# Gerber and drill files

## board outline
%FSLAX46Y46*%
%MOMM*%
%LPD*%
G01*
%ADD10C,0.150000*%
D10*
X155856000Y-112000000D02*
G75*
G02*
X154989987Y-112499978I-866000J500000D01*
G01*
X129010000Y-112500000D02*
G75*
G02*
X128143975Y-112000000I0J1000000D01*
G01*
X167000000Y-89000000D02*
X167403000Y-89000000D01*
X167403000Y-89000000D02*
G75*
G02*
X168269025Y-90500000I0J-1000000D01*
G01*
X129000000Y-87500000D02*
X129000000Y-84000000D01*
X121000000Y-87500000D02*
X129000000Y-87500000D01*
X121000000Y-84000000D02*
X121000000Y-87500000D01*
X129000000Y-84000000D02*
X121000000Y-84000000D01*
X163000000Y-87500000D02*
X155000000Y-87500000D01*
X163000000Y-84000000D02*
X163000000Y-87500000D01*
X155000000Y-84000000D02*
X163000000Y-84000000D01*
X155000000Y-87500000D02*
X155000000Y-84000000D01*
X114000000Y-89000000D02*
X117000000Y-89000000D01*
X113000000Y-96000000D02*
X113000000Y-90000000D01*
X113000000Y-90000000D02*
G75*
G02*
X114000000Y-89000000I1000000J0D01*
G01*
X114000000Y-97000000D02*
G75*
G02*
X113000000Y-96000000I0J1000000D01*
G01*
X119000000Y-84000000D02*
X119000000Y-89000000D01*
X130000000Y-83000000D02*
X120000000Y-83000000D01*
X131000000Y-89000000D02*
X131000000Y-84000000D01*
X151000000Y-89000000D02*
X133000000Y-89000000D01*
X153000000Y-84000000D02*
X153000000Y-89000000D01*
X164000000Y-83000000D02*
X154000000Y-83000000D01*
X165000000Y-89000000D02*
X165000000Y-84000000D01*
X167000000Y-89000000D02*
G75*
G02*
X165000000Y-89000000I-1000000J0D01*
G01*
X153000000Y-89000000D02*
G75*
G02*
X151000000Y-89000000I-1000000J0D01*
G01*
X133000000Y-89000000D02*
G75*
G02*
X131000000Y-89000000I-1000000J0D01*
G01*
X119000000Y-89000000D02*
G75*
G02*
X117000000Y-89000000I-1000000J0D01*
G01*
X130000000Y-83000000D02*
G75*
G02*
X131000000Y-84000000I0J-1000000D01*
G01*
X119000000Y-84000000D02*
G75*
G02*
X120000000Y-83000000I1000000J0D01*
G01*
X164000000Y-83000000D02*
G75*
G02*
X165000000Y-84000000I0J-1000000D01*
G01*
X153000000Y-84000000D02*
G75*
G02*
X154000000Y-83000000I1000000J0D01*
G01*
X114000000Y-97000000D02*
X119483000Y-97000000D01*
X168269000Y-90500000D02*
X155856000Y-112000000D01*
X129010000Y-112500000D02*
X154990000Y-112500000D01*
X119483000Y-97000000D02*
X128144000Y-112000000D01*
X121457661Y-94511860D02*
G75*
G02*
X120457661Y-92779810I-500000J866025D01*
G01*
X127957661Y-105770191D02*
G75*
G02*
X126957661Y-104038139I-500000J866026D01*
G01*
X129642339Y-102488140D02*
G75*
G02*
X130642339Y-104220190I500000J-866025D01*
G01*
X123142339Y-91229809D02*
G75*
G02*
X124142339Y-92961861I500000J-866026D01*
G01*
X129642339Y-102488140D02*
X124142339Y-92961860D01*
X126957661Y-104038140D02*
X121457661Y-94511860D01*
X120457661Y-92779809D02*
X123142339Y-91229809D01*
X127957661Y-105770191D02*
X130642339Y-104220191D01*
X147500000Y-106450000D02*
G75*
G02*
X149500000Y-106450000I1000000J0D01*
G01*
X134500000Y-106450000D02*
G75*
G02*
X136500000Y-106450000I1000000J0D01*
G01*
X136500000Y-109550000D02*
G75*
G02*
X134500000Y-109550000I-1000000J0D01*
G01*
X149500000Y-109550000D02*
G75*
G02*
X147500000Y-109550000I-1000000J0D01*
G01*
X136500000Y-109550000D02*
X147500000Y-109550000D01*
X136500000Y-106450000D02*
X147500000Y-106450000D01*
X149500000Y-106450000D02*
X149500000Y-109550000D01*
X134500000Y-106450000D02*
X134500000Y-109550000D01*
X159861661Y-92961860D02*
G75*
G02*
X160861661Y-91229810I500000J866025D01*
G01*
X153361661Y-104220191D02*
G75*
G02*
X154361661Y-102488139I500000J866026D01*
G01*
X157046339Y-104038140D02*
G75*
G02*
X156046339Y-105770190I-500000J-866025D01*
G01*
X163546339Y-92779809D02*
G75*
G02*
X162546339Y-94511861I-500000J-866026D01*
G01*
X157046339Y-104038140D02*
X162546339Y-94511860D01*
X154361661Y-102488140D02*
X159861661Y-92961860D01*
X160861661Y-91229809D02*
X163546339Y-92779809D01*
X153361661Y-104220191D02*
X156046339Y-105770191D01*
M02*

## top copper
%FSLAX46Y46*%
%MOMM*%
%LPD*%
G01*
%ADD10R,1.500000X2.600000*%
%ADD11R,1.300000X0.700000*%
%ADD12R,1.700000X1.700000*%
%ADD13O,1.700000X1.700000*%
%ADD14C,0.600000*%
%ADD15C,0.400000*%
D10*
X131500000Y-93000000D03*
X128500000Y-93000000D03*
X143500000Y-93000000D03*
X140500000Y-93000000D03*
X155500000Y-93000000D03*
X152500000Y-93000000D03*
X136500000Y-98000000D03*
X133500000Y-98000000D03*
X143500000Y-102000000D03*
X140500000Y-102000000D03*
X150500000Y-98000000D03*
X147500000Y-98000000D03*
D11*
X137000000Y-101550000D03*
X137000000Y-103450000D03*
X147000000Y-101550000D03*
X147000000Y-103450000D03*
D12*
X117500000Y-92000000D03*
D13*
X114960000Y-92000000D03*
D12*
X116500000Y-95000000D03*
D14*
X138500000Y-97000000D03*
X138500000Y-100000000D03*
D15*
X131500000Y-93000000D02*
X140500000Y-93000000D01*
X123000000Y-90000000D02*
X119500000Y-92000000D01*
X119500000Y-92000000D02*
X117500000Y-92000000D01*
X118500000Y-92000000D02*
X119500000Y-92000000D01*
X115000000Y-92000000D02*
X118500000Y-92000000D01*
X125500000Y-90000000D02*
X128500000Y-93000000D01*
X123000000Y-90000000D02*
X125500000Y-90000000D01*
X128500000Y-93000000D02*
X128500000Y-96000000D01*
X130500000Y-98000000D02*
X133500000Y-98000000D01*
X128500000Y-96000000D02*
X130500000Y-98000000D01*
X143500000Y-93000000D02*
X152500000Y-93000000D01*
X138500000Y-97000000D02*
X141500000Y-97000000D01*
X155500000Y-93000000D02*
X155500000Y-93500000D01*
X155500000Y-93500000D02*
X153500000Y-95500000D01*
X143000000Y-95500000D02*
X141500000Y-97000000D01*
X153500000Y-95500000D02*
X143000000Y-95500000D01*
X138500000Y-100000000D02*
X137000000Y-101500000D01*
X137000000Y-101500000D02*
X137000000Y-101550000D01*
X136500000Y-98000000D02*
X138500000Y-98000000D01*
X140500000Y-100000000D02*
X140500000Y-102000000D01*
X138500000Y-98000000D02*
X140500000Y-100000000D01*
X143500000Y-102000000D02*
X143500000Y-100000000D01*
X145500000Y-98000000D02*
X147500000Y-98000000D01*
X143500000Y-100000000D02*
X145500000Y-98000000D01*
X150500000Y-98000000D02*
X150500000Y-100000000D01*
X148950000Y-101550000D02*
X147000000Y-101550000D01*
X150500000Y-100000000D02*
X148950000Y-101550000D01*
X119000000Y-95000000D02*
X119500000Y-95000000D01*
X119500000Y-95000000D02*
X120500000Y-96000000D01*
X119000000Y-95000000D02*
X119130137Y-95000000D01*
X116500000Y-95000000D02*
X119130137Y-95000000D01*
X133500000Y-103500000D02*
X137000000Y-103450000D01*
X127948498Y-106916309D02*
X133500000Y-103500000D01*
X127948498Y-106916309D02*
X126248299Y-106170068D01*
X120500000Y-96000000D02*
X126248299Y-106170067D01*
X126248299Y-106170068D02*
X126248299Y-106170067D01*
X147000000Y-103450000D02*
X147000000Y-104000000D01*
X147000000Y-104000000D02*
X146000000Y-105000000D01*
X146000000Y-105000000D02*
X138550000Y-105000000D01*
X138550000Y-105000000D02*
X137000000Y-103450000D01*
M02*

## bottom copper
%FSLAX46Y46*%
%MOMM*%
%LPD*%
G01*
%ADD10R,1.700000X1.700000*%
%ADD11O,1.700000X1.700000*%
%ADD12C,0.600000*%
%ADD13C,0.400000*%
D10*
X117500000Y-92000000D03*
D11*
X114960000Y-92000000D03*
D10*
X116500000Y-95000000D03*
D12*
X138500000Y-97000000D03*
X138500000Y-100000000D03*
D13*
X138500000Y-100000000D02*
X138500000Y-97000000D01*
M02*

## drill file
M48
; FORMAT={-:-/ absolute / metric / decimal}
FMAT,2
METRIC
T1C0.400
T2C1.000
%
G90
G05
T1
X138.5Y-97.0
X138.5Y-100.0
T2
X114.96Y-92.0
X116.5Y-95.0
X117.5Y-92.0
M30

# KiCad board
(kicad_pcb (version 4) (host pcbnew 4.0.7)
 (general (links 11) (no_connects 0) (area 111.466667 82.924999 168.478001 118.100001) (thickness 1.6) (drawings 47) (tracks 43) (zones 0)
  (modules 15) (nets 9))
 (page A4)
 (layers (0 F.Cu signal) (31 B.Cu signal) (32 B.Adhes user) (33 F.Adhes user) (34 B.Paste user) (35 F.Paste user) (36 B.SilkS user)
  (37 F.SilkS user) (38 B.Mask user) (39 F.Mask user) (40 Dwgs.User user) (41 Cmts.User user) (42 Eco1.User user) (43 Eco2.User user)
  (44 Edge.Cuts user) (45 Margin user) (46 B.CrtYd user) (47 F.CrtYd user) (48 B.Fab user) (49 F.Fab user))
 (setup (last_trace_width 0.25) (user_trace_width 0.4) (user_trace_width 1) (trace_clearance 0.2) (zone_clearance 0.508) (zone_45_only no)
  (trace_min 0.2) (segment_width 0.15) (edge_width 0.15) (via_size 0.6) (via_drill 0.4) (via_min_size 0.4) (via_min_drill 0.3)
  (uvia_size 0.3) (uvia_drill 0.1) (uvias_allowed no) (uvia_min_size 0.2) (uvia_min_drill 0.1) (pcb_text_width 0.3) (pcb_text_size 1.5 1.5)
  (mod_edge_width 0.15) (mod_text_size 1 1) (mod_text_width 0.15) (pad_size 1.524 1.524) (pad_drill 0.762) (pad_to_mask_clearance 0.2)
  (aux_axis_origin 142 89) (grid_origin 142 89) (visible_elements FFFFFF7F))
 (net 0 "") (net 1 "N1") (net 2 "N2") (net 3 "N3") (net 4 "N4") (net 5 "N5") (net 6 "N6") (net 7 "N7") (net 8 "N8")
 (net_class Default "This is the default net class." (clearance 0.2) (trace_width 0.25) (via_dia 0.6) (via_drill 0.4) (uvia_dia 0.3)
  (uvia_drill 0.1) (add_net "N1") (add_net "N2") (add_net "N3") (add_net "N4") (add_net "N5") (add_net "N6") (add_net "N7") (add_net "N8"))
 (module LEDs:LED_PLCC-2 (layer F.Cu) (at 130 93 180)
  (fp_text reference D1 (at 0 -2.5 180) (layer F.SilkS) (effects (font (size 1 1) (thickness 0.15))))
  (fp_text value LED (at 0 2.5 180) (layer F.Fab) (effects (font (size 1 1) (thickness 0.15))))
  (pad 1 smd rect (at -1.5 0 180) (size 1.5 2.6) (layers F.Cu F.Paste F.Mask) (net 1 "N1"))
  (pad 2 smd rect (at 1.5 0 180) (size 1.5 2.6) (layers F.Cu F.Paste F.Mask) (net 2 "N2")))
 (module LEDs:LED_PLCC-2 (layer F.Cu) (at 142 93 180)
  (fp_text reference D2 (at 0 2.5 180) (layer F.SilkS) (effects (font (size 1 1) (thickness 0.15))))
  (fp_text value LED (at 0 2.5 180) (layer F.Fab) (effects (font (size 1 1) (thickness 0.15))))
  (pad 1 smd rect (at -1.5 0 180) (size 1.5 2.6) (layers F.Cu F.Paste F.Mask) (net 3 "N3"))
  (pad 2 smd rect (at 1.5 0 180) (size 1.5 2.6) (layers F.Cu F.Paste F.Mask) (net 1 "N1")))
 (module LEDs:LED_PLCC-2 (layer F.Cu) (at 154 93 180)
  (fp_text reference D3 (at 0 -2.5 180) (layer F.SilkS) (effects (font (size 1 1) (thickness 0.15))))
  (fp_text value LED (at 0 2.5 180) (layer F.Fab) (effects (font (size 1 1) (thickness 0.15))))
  (pad 1 smd rect (at -1.5 0 180) (size 1.5 2.6) (layers F.Cu F.Paste F.Mask) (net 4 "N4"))
  (pad 2 smd rect (at 1.5 0 180) (size 1.5 2.6) (layers F.Cu F.Paste F.Mask) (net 3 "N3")))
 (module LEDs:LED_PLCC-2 (layer F.Cu) (at 135 98 180)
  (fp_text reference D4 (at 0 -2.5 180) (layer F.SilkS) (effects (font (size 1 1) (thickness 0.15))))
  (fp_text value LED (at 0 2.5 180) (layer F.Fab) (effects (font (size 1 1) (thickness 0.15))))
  (pad 1 smd rect (at -1.5 0 180) (size 1.5 2.6) (layers F.Cu F.Paste F.Mask) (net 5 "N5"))
  (pad 2 smd rect (at 1.5 0 180) (size 1.5 2.6) (layers F.Cu F.Paste F.Mask) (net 2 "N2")))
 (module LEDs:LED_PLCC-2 (layer F.Cu) (at 142 102 180)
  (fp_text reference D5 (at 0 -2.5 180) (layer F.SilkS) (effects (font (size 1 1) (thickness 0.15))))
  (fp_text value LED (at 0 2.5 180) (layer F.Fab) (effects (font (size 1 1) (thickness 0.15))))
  (pad 1 smd rect (at -1.5 0 180) (size 1.5 2.6) (layers F.Cu F.Paste F.Mask) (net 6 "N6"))
  (pad 2 smd rect (at 1.5 0 180) (size 1.5 2.6) (layers F.Cu F.Paste F.Mask) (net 5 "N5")))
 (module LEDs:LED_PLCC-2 (layer F.Cu) (at 149 98 180)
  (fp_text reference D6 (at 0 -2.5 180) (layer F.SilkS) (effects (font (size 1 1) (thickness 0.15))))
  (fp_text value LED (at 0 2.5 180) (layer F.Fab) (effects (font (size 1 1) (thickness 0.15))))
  (pad 1 smd rect (at -1.5 0 180) (size 1.5 2.6) (layers F.Cu F.Paste F.Mask) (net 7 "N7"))
  (pad 2 smd rect (at 1.5 0 180) (size 1.5 2.6) (layers F.Cu F.Paste F.Mask) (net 6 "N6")))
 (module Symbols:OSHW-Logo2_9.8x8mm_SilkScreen (layer B.Cu) (at 142 100 180)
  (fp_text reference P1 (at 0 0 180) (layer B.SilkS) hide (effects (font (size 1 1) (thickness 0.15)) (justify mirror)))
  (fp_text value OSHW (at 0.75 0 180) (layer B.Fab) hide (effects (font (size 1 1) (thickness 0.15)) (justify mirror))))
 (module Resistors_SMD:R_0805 (layer F.Cu) (at 137 102.5 270)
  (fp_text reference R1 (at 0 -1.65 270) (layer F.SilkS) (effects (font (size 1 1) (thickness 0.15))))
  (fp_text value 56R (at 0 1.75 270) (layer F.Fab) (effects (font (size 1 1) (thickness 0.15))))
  (pad 1 smd rect (at -0.95 0 270) (size 0.7 1.3) (layers F.Cu F.Paste F.Mask) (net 4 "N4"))
  (pad 2 smd rect (at 0.95 0 270) (size 0.7 1.3) (layers F.Cu F.Paste F.Mask) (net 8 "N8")))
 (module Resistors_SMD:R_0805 (layer F.Cu) (at 147 102.5 270)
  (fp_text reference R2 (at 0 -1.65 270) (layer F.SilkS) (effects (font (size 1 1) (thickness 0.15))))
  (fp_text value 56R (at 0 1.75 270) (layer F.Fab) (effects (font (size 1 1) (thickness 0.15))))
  (pad 1 smd rect (at -0.95 0 270) (size 0.7 1.3) (layers F.Cu F.Paste F.Mask) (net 7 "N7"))
  (pad 2 smd rect (at 0.95 0 270) (size 0.7 1.3) (layers F.Cu F.Paste F.Mask) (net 8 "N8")))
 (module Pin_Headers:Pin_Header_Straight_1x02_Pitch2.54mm (layer F.Cu) (at 117.5 92 270)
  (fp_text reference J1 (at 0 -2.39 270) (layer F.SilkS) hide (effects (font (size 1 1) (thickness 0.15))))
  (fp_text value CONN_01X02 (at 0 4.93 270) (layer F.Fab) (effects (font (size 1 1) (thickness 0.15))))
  (pad 1 thru_hole rect (at 0 0 270) (size 1.7 1.7) (drill 1) (layers *.Cu *.Mask) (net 2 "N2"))
  (pad 2 thru_hole oval (at 0 2.54 270) (size 1.7 1.7) (drill 1) (layers *.Cu *.Mask) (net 2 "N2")))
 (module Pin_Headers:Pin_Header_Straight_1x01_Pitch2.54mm (layer F.Cu) (at 116.5 95)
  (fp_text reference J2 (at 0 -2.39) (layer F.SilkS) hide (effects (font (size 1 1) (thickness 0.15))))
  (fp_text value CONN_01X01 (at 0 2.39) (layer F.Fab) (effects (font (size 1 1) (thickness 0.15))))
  (pad 1 thru_hole rect (at 0 0) (size 1.7 1.7) (drill 1) (layers *.Cu *.Mask) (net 8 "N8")))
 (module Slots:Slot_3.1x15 (layer F.Cu) (at 125.55 98.5 120)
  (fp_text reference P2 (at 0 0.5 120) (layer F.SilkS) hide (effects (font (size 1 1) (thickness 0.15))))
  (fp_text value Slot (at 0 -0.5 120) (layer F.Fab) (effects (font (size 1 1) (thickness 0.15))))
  (fp_arc (start 6.5 -1.55) (end 5.5 -1.55) (angle 180) (layer Edge.Cuts) (width 0.15))
  (fp_arc (start -6.5 -1.55) (end -7.5 -1.55) (angle 180) (layer Edge.Cuts) (width 0.15))
  (fp_arc (start -6.5 1.55) (end -5.5 1.55) (angle 180) (layer Edge.Cuts) (width 0.15))
  (fp_arc (start 6.5 1.55) (end 7.5 1.55) (angle 180) (layer Edge.Cuts) (width 0.15))
  (fp_line (start -5.5 1.55) (end 5.5 1.55) (layer Edge.Cuts) (width 0.15))
  (fp_line (start -5.5 -1.55) (end 5.5 -1.55) (layer Edge.Cuts) (width 0.15))
  (fp_line (start 7.5 -1.55) (end 7.5 1.55) (layer Edge.Cuts) (width 0.15))
  (fp_line (start -7.5 -1.55) (end -7.5 1.55) (layer Edge.Cuts) (width 0.15)))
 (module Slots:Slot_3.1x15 (layer F.Cu) (at 142 108)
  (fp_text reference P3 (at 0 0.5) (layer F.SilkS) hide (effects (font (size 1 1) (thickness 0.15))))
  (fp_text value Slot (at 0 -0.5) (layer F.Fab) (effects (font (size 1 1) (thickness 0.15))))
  (fp_arc (start 6.5 -1.55) (end 5.5 -1.55) (angle 180) (layer Edge.Cuts) (width 0.15))
  (fp_arc (start -6.5 -1.55) (end -7.5 -1.55) (angle 180) (layer Edge.Cuts) (width 0.15))
  (fp_arc (start -6.5 1.55) (end -5.5 1.55) (angle 180) (layer Edge.Cuts) (width 0.15))
  (fp_arc (start 6.5 1.55) (end 7.5 1.55) (angle 180) (layer Edge.Cuts) (width 0.15))
  (fp_line (start -5.5 1.55) (end 5.5 1.55) (layer Edge.Cuts) (width 0.15))
  (fp_line (start -5.5 -1.55) (end 5.5 -1.55) (layer Edge.Cuts) (width 0.15))
  (fp_line (start 7.5 -1.55) (end 7.5 1.55) (layer Edge.Cuts) (width 0.15))
  (fp_line (start -7.5 -1.55) (end -7.5 1.55) (layer Edge.Cuts) (width 0.15)))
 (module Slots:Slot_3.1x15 (layer F.Cu) (at 158.454 98.5 60)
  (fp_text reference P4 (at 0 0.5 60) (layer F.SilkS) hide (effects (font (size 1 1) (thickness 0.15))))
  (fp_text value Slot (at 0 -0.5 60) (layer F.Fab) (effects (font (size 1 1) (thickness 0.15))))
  (fp_arc (start 6.5 -1.55) (end 5.5 -1.55) (angle 180) (layer Edge.Cuts) (width 0.15))
  (fp_arc (start -6.5 -1.55) (end -7.5 -1.55) (angle 180) (layer Edge.Cuts) (width 0.15))
  (fp_arc (start -6.5 1.55) (end -5.5 1.55) (angle 180) (layer Edge.Cuts) (width 0.15))
  (fp_arc (start 6.5 1.55) (end 7.5 1.55) (angle 180) (layer Edge.Cuts) (width 0.15))
  (fp_line (start -5.5 1.55) (end 5.5 1.55) (layer Edge.Cuts) (width 0.15))
  (fp_line (start -5.5 -1.55) (end 5.5 -1.55) (layer Edge.Cuts) (width 0.15))
  (fp_line (start 7.5 -1.55) (end 7.5 1.55) (layer Edge.Cuts) (width 0.15))
  (fp_line (start -7.5 -1.55) (end -7.5 1.55) (layer Edge.Cuts) (width 0.15)))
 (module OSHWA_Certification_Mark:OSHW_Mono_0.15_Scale (layer F.Cu) (at 142 96.5)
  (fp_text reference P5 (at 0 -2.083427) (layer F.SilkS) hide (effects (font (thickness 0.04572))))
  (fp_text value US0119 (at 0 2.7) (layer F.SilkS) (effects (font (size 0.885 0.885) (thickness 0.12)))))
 (gr_arc (start 154.99 111.5) (end 155.856 112) (angle 60) (layer Edge.Cuts) (width 0.15))
 (gr_arc (start 129.01 111.5) (end 129.01 112.5) (angle 60) (layer Edge.Cuts) (width 0.15))
 (gr_line (start 167 89) (end 167.403 89) (angle 90) (layer Edge.Cuts) (width 0.15))
 (gr_arc (start 167.403 90) (end 167.403 89) (angle 120) (layer Edge.Cuts) (width 0.15))
 (gr_line (start 129 87.5) (end 129 84) (angle 90) (layer Edge.Cuts) (width 0.15))
 (gr_line (start 121 87.5) (end 129 87.5) (angle 90) (layer Edge.Cuts) (width 0.15))
 (gr_line (start 121 84) (end 121 87.5) (angle 90) (layer Edge.Cuts) (width 0.15))
 (gr_line (start 129 84) (end 121 84) (angle 90) (layer Edge.Cuts) (width 0.15))
 (gr_line (start 163 87.5) (end 155 87.5) (angle 90) (layer Edge.Cuts) (width 0.15))
 (gr_line (start 163 84) (end 163 87.5) (angle 90) (layer Edge.Cuts) (width 0.15))
 (gr_line (start 155 84) (end 163 84) (angle 90) (layer Edge.Cuts) (width 0.15))
 (gr_line (start 155 87.5) (end 155 84) (angle 90) (layer Edge.Cuts) (width 0.15))
 (gr_line (start 114 89) (end 117 89) (angle 90) (layer Edge.Cuts) (width 0.15))
 (gr_line (start 113 96) (end 113 90) (angle 90) (layer Edge.Cuts) (width 0.15))
 (gr_arc (start 114 90) (end 113 90) (angle 90) (layer Edge.Cuts) (width 0.15))
 (gr_arc (start 114 96) (end 114 97) (angle 90) (layer Edge.Cuts) (width 0.15))
 (gr_line (start 119 84) (end 119 89) (angle 90) (layer Edge.Cuts) (width 0.15))
 (gr_line (start 130 83) (end 120 83) (angle 90) (layer Edge.Cuts) (width 0.15))
 (gr_line (start 131 89) (end 131 84) (angle 90) (layer Edge.Cuts) (width 0.15))
 (gr_line (start 151 89) (end 133 89) (angle 90) (layer Edge.Cuts) (width 0.15))
 (gr_line (start 153 84) (end 153 89) (angle 90) (layer Edge.Cuts) (width 0.15))
 (gr_line (start 164 83) (end 154 83) (angle 90) (layer Edge.Cuts) (width 0.15))
 (gr_line (start 165 89) (end 165 84) (angle 90) (layer Edge.Cuts) (width 0.15))
 (gr_arc (start 166 89) (end 167 89) (angle 180) (layer Edge.Cuts) (width 0.15))
 (gr_arc (start 152 89) (end 153 89) (angle 180) (layer Edge.Cuts) (width 0.15))
 (gr_arc (start 132 89) (end 133 89) (angle 180) (layer Edge.Cuts) (width 0.15))
 (gr_arc (start 118 89) (end 119 89) (angle 180) (layer Edge.Cuts) (width 0.15))
 (gr_arc (start 130 84) (end 130 83) (angle 90) (layer Edge.Cuts) (width 0.15))
 (gr_arc (start 120 84) (end 119 84) (angle 90) (layer Edge.Cuts) (width 0.15))
 (gr_arc (start 164 84) (end 164 83) (angle 90) (layer Edge.Cuts) (width 0.15))
 (gr_arc (start 154 84) (end 153 84) (angle 90) (layer Edge.Cuts) (width 0.15))
 (gr_line (start 114 97) (end 119.483 97) (angle 90) (layer Edge.Cuts) (width 0.15))
 (gr_line (start 168.269 90.5) (end 155.856 112) (angle 90) (layer Edge.Cuts) (width 0.15))
 (gr_line (start 129.01 112.5) (end 154.99 112.5) (angle 90) (layer Edge.Cuts) (width 0.15))
 (gr_line (start 119.483 97) (end 128.144 112) (angle 90) (layer Edge.Cuts) (width 0.15))
 (segment (start 131.5 93) (end 140.5 93) (width 0.4) (layer F.Cu) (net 1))
 (segment (start 123 90) (end 119.5 92) (width 0.4) (layer F.Cu) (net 2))
 (segment (start 119.5 92) (end 117.5 92) (width 0.4) (layer F.Cu) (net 2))
 (segment (start 118.5 92) (end 119.5 92) (width 0.4) (layer F.Cu) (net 2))
 (segment (start 115 92) (end 118.5 92) (width 0.4) (layer F.Cu) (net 2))
 (segment (start 125.5 90) (end 128.5 93) (width 0.4) (layer F.Cu) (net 2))
 (segment (start 123 90) (end 125.5 90) (width 0.4) (layer F.Cu) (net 2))
 (segment (start 128.5 93) (end 128.5 96) (width 0.4) (layer F.Cu) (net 2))
 (segment (start 130.5 98) (end 133.5 98) (width 0.4) (layer F.Cu) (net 2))
 (segment (start 128.5 96) (end 130.5 98) (width 0.4) (layer F.Cu) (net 2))
 (segment (start 143.5 93) (end 152.5 93) (width 0.4) (layer F.Cu) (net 3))
 (segment (start 138.5 100) (end 138.5 97) (width 0.4) (layer B.Cu) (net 4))
 (segment (start 138.5 97) (end 141.5 97) (width 0.4) (layer F.Cu) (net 4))
 (via (at 138.5 97) (size 0.6) (drill 0.4) (layers F.Cu B.Cu) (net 4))
 (segment (start 155.5 93) (end 155.5 93.5) (width 0.4) (layer F.Cu) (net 4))
 (segment (start 155.5 93.5) (end 153.5 95.5) (width 0.4) (layer F.Cu) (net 4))
 (segment (start 143 95.5) (end 141.5 97) (width 0.4) (layer F.Cu) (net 4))
 (segment (start 153.5 95.5) (end 143 95.5) (width 0.4) (layer F.Cu) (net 4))
 (via (at 138.5 100) (size 0.6) (drill 0.4) (layers F.Cu B.Cu) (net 4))
 (segment (start 138.5 100) (end 137 101.5) (width 0.4) (layer F.Cu) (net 4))
 (segment (start 137 101.5) (end 137 101.55) (width 0.4) (layer F.Cu) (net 4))
 (segment (start 136.5 98) (end 138.5 98) (width 0.4) (layer F.Cu) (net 5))
 (segment (start 140.5 100) (end 140.5 102) (width 0.4) (layer F.Cu) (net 5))
 (segment (start 138.5 98) (end 140.5 100) (width 0.4) (layer F.Cu) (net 5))
 (segment (start 143.5 102) (end 143.5 100) (width 0.4) (layer F.Cu) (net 6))
 (segment (start 145.5 98) (end 147.5 98) (width 0.4) (layer F.Cu) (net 6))
 (segment (start 143.5 100) (end 145.5 98) (width 0.4) (layer F.Cu) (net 6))
 (segment (start 150.5 98) (end 150.5 100) (width 0.4) (layer F.Cu) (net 7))
 (segment (start 148.95 101.55) (end 147 101.55) (width 0.4) (layer F.Cu) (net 7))
 (segment (start 150.5 100) (end 148.95 101.55) (width 0.4) (layer F.Cu) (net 7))
 (segment (start 119 95) (end 119.5 95) (width 0.4) (layer F.Cu) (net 8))
 (segment (start 119.5 95) (end 120.5 96) (width 0.4) (layer F.Cu) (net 8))
 (segment (start 119 95) (end 119.130137 95) (width 0.4) (layer F.Cu) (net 8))
 (segment (start 116.5 95) (end 119.130137 95) (width 0.4) (layer F.Cu) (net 8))
 (segment (start 133.5 103.5) (end 137 103.45) (width 0.4) (layer F.Cu) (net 8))
 (segment (start 127.948498 106.916309) (end 133.5 103.5) (width 0.4) (layer F.Cu) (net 8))
 (segment (start 127.948498 106.916309) (end 126.248299 106.170068) (width 0.4) (layer F.Cu) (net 8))
 (segment (start 120.5 96) (end 126.248299 106.170067) (width 0.4) (layer F.Cu) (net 8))
 (segment (start 126.248299 106.170068) (end 126.248299 106.170067) (width 0.4) (layer F.Cu) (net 8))
 (segment (start 147 103.45) (end 147 104) (width 0.4) (layer F.Cu) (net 8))
 (segment (start 147 104) (end 146 105) (width 0.4) (layer F.Cu) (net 8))
 (segment (start 146 105) (end 138.55 105) (width 0.4) (layer F.Cu) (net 8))
 (segment (start 138.55 105) (end 137 103.45) (width 0.4) (layer F.Cu) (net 8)))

